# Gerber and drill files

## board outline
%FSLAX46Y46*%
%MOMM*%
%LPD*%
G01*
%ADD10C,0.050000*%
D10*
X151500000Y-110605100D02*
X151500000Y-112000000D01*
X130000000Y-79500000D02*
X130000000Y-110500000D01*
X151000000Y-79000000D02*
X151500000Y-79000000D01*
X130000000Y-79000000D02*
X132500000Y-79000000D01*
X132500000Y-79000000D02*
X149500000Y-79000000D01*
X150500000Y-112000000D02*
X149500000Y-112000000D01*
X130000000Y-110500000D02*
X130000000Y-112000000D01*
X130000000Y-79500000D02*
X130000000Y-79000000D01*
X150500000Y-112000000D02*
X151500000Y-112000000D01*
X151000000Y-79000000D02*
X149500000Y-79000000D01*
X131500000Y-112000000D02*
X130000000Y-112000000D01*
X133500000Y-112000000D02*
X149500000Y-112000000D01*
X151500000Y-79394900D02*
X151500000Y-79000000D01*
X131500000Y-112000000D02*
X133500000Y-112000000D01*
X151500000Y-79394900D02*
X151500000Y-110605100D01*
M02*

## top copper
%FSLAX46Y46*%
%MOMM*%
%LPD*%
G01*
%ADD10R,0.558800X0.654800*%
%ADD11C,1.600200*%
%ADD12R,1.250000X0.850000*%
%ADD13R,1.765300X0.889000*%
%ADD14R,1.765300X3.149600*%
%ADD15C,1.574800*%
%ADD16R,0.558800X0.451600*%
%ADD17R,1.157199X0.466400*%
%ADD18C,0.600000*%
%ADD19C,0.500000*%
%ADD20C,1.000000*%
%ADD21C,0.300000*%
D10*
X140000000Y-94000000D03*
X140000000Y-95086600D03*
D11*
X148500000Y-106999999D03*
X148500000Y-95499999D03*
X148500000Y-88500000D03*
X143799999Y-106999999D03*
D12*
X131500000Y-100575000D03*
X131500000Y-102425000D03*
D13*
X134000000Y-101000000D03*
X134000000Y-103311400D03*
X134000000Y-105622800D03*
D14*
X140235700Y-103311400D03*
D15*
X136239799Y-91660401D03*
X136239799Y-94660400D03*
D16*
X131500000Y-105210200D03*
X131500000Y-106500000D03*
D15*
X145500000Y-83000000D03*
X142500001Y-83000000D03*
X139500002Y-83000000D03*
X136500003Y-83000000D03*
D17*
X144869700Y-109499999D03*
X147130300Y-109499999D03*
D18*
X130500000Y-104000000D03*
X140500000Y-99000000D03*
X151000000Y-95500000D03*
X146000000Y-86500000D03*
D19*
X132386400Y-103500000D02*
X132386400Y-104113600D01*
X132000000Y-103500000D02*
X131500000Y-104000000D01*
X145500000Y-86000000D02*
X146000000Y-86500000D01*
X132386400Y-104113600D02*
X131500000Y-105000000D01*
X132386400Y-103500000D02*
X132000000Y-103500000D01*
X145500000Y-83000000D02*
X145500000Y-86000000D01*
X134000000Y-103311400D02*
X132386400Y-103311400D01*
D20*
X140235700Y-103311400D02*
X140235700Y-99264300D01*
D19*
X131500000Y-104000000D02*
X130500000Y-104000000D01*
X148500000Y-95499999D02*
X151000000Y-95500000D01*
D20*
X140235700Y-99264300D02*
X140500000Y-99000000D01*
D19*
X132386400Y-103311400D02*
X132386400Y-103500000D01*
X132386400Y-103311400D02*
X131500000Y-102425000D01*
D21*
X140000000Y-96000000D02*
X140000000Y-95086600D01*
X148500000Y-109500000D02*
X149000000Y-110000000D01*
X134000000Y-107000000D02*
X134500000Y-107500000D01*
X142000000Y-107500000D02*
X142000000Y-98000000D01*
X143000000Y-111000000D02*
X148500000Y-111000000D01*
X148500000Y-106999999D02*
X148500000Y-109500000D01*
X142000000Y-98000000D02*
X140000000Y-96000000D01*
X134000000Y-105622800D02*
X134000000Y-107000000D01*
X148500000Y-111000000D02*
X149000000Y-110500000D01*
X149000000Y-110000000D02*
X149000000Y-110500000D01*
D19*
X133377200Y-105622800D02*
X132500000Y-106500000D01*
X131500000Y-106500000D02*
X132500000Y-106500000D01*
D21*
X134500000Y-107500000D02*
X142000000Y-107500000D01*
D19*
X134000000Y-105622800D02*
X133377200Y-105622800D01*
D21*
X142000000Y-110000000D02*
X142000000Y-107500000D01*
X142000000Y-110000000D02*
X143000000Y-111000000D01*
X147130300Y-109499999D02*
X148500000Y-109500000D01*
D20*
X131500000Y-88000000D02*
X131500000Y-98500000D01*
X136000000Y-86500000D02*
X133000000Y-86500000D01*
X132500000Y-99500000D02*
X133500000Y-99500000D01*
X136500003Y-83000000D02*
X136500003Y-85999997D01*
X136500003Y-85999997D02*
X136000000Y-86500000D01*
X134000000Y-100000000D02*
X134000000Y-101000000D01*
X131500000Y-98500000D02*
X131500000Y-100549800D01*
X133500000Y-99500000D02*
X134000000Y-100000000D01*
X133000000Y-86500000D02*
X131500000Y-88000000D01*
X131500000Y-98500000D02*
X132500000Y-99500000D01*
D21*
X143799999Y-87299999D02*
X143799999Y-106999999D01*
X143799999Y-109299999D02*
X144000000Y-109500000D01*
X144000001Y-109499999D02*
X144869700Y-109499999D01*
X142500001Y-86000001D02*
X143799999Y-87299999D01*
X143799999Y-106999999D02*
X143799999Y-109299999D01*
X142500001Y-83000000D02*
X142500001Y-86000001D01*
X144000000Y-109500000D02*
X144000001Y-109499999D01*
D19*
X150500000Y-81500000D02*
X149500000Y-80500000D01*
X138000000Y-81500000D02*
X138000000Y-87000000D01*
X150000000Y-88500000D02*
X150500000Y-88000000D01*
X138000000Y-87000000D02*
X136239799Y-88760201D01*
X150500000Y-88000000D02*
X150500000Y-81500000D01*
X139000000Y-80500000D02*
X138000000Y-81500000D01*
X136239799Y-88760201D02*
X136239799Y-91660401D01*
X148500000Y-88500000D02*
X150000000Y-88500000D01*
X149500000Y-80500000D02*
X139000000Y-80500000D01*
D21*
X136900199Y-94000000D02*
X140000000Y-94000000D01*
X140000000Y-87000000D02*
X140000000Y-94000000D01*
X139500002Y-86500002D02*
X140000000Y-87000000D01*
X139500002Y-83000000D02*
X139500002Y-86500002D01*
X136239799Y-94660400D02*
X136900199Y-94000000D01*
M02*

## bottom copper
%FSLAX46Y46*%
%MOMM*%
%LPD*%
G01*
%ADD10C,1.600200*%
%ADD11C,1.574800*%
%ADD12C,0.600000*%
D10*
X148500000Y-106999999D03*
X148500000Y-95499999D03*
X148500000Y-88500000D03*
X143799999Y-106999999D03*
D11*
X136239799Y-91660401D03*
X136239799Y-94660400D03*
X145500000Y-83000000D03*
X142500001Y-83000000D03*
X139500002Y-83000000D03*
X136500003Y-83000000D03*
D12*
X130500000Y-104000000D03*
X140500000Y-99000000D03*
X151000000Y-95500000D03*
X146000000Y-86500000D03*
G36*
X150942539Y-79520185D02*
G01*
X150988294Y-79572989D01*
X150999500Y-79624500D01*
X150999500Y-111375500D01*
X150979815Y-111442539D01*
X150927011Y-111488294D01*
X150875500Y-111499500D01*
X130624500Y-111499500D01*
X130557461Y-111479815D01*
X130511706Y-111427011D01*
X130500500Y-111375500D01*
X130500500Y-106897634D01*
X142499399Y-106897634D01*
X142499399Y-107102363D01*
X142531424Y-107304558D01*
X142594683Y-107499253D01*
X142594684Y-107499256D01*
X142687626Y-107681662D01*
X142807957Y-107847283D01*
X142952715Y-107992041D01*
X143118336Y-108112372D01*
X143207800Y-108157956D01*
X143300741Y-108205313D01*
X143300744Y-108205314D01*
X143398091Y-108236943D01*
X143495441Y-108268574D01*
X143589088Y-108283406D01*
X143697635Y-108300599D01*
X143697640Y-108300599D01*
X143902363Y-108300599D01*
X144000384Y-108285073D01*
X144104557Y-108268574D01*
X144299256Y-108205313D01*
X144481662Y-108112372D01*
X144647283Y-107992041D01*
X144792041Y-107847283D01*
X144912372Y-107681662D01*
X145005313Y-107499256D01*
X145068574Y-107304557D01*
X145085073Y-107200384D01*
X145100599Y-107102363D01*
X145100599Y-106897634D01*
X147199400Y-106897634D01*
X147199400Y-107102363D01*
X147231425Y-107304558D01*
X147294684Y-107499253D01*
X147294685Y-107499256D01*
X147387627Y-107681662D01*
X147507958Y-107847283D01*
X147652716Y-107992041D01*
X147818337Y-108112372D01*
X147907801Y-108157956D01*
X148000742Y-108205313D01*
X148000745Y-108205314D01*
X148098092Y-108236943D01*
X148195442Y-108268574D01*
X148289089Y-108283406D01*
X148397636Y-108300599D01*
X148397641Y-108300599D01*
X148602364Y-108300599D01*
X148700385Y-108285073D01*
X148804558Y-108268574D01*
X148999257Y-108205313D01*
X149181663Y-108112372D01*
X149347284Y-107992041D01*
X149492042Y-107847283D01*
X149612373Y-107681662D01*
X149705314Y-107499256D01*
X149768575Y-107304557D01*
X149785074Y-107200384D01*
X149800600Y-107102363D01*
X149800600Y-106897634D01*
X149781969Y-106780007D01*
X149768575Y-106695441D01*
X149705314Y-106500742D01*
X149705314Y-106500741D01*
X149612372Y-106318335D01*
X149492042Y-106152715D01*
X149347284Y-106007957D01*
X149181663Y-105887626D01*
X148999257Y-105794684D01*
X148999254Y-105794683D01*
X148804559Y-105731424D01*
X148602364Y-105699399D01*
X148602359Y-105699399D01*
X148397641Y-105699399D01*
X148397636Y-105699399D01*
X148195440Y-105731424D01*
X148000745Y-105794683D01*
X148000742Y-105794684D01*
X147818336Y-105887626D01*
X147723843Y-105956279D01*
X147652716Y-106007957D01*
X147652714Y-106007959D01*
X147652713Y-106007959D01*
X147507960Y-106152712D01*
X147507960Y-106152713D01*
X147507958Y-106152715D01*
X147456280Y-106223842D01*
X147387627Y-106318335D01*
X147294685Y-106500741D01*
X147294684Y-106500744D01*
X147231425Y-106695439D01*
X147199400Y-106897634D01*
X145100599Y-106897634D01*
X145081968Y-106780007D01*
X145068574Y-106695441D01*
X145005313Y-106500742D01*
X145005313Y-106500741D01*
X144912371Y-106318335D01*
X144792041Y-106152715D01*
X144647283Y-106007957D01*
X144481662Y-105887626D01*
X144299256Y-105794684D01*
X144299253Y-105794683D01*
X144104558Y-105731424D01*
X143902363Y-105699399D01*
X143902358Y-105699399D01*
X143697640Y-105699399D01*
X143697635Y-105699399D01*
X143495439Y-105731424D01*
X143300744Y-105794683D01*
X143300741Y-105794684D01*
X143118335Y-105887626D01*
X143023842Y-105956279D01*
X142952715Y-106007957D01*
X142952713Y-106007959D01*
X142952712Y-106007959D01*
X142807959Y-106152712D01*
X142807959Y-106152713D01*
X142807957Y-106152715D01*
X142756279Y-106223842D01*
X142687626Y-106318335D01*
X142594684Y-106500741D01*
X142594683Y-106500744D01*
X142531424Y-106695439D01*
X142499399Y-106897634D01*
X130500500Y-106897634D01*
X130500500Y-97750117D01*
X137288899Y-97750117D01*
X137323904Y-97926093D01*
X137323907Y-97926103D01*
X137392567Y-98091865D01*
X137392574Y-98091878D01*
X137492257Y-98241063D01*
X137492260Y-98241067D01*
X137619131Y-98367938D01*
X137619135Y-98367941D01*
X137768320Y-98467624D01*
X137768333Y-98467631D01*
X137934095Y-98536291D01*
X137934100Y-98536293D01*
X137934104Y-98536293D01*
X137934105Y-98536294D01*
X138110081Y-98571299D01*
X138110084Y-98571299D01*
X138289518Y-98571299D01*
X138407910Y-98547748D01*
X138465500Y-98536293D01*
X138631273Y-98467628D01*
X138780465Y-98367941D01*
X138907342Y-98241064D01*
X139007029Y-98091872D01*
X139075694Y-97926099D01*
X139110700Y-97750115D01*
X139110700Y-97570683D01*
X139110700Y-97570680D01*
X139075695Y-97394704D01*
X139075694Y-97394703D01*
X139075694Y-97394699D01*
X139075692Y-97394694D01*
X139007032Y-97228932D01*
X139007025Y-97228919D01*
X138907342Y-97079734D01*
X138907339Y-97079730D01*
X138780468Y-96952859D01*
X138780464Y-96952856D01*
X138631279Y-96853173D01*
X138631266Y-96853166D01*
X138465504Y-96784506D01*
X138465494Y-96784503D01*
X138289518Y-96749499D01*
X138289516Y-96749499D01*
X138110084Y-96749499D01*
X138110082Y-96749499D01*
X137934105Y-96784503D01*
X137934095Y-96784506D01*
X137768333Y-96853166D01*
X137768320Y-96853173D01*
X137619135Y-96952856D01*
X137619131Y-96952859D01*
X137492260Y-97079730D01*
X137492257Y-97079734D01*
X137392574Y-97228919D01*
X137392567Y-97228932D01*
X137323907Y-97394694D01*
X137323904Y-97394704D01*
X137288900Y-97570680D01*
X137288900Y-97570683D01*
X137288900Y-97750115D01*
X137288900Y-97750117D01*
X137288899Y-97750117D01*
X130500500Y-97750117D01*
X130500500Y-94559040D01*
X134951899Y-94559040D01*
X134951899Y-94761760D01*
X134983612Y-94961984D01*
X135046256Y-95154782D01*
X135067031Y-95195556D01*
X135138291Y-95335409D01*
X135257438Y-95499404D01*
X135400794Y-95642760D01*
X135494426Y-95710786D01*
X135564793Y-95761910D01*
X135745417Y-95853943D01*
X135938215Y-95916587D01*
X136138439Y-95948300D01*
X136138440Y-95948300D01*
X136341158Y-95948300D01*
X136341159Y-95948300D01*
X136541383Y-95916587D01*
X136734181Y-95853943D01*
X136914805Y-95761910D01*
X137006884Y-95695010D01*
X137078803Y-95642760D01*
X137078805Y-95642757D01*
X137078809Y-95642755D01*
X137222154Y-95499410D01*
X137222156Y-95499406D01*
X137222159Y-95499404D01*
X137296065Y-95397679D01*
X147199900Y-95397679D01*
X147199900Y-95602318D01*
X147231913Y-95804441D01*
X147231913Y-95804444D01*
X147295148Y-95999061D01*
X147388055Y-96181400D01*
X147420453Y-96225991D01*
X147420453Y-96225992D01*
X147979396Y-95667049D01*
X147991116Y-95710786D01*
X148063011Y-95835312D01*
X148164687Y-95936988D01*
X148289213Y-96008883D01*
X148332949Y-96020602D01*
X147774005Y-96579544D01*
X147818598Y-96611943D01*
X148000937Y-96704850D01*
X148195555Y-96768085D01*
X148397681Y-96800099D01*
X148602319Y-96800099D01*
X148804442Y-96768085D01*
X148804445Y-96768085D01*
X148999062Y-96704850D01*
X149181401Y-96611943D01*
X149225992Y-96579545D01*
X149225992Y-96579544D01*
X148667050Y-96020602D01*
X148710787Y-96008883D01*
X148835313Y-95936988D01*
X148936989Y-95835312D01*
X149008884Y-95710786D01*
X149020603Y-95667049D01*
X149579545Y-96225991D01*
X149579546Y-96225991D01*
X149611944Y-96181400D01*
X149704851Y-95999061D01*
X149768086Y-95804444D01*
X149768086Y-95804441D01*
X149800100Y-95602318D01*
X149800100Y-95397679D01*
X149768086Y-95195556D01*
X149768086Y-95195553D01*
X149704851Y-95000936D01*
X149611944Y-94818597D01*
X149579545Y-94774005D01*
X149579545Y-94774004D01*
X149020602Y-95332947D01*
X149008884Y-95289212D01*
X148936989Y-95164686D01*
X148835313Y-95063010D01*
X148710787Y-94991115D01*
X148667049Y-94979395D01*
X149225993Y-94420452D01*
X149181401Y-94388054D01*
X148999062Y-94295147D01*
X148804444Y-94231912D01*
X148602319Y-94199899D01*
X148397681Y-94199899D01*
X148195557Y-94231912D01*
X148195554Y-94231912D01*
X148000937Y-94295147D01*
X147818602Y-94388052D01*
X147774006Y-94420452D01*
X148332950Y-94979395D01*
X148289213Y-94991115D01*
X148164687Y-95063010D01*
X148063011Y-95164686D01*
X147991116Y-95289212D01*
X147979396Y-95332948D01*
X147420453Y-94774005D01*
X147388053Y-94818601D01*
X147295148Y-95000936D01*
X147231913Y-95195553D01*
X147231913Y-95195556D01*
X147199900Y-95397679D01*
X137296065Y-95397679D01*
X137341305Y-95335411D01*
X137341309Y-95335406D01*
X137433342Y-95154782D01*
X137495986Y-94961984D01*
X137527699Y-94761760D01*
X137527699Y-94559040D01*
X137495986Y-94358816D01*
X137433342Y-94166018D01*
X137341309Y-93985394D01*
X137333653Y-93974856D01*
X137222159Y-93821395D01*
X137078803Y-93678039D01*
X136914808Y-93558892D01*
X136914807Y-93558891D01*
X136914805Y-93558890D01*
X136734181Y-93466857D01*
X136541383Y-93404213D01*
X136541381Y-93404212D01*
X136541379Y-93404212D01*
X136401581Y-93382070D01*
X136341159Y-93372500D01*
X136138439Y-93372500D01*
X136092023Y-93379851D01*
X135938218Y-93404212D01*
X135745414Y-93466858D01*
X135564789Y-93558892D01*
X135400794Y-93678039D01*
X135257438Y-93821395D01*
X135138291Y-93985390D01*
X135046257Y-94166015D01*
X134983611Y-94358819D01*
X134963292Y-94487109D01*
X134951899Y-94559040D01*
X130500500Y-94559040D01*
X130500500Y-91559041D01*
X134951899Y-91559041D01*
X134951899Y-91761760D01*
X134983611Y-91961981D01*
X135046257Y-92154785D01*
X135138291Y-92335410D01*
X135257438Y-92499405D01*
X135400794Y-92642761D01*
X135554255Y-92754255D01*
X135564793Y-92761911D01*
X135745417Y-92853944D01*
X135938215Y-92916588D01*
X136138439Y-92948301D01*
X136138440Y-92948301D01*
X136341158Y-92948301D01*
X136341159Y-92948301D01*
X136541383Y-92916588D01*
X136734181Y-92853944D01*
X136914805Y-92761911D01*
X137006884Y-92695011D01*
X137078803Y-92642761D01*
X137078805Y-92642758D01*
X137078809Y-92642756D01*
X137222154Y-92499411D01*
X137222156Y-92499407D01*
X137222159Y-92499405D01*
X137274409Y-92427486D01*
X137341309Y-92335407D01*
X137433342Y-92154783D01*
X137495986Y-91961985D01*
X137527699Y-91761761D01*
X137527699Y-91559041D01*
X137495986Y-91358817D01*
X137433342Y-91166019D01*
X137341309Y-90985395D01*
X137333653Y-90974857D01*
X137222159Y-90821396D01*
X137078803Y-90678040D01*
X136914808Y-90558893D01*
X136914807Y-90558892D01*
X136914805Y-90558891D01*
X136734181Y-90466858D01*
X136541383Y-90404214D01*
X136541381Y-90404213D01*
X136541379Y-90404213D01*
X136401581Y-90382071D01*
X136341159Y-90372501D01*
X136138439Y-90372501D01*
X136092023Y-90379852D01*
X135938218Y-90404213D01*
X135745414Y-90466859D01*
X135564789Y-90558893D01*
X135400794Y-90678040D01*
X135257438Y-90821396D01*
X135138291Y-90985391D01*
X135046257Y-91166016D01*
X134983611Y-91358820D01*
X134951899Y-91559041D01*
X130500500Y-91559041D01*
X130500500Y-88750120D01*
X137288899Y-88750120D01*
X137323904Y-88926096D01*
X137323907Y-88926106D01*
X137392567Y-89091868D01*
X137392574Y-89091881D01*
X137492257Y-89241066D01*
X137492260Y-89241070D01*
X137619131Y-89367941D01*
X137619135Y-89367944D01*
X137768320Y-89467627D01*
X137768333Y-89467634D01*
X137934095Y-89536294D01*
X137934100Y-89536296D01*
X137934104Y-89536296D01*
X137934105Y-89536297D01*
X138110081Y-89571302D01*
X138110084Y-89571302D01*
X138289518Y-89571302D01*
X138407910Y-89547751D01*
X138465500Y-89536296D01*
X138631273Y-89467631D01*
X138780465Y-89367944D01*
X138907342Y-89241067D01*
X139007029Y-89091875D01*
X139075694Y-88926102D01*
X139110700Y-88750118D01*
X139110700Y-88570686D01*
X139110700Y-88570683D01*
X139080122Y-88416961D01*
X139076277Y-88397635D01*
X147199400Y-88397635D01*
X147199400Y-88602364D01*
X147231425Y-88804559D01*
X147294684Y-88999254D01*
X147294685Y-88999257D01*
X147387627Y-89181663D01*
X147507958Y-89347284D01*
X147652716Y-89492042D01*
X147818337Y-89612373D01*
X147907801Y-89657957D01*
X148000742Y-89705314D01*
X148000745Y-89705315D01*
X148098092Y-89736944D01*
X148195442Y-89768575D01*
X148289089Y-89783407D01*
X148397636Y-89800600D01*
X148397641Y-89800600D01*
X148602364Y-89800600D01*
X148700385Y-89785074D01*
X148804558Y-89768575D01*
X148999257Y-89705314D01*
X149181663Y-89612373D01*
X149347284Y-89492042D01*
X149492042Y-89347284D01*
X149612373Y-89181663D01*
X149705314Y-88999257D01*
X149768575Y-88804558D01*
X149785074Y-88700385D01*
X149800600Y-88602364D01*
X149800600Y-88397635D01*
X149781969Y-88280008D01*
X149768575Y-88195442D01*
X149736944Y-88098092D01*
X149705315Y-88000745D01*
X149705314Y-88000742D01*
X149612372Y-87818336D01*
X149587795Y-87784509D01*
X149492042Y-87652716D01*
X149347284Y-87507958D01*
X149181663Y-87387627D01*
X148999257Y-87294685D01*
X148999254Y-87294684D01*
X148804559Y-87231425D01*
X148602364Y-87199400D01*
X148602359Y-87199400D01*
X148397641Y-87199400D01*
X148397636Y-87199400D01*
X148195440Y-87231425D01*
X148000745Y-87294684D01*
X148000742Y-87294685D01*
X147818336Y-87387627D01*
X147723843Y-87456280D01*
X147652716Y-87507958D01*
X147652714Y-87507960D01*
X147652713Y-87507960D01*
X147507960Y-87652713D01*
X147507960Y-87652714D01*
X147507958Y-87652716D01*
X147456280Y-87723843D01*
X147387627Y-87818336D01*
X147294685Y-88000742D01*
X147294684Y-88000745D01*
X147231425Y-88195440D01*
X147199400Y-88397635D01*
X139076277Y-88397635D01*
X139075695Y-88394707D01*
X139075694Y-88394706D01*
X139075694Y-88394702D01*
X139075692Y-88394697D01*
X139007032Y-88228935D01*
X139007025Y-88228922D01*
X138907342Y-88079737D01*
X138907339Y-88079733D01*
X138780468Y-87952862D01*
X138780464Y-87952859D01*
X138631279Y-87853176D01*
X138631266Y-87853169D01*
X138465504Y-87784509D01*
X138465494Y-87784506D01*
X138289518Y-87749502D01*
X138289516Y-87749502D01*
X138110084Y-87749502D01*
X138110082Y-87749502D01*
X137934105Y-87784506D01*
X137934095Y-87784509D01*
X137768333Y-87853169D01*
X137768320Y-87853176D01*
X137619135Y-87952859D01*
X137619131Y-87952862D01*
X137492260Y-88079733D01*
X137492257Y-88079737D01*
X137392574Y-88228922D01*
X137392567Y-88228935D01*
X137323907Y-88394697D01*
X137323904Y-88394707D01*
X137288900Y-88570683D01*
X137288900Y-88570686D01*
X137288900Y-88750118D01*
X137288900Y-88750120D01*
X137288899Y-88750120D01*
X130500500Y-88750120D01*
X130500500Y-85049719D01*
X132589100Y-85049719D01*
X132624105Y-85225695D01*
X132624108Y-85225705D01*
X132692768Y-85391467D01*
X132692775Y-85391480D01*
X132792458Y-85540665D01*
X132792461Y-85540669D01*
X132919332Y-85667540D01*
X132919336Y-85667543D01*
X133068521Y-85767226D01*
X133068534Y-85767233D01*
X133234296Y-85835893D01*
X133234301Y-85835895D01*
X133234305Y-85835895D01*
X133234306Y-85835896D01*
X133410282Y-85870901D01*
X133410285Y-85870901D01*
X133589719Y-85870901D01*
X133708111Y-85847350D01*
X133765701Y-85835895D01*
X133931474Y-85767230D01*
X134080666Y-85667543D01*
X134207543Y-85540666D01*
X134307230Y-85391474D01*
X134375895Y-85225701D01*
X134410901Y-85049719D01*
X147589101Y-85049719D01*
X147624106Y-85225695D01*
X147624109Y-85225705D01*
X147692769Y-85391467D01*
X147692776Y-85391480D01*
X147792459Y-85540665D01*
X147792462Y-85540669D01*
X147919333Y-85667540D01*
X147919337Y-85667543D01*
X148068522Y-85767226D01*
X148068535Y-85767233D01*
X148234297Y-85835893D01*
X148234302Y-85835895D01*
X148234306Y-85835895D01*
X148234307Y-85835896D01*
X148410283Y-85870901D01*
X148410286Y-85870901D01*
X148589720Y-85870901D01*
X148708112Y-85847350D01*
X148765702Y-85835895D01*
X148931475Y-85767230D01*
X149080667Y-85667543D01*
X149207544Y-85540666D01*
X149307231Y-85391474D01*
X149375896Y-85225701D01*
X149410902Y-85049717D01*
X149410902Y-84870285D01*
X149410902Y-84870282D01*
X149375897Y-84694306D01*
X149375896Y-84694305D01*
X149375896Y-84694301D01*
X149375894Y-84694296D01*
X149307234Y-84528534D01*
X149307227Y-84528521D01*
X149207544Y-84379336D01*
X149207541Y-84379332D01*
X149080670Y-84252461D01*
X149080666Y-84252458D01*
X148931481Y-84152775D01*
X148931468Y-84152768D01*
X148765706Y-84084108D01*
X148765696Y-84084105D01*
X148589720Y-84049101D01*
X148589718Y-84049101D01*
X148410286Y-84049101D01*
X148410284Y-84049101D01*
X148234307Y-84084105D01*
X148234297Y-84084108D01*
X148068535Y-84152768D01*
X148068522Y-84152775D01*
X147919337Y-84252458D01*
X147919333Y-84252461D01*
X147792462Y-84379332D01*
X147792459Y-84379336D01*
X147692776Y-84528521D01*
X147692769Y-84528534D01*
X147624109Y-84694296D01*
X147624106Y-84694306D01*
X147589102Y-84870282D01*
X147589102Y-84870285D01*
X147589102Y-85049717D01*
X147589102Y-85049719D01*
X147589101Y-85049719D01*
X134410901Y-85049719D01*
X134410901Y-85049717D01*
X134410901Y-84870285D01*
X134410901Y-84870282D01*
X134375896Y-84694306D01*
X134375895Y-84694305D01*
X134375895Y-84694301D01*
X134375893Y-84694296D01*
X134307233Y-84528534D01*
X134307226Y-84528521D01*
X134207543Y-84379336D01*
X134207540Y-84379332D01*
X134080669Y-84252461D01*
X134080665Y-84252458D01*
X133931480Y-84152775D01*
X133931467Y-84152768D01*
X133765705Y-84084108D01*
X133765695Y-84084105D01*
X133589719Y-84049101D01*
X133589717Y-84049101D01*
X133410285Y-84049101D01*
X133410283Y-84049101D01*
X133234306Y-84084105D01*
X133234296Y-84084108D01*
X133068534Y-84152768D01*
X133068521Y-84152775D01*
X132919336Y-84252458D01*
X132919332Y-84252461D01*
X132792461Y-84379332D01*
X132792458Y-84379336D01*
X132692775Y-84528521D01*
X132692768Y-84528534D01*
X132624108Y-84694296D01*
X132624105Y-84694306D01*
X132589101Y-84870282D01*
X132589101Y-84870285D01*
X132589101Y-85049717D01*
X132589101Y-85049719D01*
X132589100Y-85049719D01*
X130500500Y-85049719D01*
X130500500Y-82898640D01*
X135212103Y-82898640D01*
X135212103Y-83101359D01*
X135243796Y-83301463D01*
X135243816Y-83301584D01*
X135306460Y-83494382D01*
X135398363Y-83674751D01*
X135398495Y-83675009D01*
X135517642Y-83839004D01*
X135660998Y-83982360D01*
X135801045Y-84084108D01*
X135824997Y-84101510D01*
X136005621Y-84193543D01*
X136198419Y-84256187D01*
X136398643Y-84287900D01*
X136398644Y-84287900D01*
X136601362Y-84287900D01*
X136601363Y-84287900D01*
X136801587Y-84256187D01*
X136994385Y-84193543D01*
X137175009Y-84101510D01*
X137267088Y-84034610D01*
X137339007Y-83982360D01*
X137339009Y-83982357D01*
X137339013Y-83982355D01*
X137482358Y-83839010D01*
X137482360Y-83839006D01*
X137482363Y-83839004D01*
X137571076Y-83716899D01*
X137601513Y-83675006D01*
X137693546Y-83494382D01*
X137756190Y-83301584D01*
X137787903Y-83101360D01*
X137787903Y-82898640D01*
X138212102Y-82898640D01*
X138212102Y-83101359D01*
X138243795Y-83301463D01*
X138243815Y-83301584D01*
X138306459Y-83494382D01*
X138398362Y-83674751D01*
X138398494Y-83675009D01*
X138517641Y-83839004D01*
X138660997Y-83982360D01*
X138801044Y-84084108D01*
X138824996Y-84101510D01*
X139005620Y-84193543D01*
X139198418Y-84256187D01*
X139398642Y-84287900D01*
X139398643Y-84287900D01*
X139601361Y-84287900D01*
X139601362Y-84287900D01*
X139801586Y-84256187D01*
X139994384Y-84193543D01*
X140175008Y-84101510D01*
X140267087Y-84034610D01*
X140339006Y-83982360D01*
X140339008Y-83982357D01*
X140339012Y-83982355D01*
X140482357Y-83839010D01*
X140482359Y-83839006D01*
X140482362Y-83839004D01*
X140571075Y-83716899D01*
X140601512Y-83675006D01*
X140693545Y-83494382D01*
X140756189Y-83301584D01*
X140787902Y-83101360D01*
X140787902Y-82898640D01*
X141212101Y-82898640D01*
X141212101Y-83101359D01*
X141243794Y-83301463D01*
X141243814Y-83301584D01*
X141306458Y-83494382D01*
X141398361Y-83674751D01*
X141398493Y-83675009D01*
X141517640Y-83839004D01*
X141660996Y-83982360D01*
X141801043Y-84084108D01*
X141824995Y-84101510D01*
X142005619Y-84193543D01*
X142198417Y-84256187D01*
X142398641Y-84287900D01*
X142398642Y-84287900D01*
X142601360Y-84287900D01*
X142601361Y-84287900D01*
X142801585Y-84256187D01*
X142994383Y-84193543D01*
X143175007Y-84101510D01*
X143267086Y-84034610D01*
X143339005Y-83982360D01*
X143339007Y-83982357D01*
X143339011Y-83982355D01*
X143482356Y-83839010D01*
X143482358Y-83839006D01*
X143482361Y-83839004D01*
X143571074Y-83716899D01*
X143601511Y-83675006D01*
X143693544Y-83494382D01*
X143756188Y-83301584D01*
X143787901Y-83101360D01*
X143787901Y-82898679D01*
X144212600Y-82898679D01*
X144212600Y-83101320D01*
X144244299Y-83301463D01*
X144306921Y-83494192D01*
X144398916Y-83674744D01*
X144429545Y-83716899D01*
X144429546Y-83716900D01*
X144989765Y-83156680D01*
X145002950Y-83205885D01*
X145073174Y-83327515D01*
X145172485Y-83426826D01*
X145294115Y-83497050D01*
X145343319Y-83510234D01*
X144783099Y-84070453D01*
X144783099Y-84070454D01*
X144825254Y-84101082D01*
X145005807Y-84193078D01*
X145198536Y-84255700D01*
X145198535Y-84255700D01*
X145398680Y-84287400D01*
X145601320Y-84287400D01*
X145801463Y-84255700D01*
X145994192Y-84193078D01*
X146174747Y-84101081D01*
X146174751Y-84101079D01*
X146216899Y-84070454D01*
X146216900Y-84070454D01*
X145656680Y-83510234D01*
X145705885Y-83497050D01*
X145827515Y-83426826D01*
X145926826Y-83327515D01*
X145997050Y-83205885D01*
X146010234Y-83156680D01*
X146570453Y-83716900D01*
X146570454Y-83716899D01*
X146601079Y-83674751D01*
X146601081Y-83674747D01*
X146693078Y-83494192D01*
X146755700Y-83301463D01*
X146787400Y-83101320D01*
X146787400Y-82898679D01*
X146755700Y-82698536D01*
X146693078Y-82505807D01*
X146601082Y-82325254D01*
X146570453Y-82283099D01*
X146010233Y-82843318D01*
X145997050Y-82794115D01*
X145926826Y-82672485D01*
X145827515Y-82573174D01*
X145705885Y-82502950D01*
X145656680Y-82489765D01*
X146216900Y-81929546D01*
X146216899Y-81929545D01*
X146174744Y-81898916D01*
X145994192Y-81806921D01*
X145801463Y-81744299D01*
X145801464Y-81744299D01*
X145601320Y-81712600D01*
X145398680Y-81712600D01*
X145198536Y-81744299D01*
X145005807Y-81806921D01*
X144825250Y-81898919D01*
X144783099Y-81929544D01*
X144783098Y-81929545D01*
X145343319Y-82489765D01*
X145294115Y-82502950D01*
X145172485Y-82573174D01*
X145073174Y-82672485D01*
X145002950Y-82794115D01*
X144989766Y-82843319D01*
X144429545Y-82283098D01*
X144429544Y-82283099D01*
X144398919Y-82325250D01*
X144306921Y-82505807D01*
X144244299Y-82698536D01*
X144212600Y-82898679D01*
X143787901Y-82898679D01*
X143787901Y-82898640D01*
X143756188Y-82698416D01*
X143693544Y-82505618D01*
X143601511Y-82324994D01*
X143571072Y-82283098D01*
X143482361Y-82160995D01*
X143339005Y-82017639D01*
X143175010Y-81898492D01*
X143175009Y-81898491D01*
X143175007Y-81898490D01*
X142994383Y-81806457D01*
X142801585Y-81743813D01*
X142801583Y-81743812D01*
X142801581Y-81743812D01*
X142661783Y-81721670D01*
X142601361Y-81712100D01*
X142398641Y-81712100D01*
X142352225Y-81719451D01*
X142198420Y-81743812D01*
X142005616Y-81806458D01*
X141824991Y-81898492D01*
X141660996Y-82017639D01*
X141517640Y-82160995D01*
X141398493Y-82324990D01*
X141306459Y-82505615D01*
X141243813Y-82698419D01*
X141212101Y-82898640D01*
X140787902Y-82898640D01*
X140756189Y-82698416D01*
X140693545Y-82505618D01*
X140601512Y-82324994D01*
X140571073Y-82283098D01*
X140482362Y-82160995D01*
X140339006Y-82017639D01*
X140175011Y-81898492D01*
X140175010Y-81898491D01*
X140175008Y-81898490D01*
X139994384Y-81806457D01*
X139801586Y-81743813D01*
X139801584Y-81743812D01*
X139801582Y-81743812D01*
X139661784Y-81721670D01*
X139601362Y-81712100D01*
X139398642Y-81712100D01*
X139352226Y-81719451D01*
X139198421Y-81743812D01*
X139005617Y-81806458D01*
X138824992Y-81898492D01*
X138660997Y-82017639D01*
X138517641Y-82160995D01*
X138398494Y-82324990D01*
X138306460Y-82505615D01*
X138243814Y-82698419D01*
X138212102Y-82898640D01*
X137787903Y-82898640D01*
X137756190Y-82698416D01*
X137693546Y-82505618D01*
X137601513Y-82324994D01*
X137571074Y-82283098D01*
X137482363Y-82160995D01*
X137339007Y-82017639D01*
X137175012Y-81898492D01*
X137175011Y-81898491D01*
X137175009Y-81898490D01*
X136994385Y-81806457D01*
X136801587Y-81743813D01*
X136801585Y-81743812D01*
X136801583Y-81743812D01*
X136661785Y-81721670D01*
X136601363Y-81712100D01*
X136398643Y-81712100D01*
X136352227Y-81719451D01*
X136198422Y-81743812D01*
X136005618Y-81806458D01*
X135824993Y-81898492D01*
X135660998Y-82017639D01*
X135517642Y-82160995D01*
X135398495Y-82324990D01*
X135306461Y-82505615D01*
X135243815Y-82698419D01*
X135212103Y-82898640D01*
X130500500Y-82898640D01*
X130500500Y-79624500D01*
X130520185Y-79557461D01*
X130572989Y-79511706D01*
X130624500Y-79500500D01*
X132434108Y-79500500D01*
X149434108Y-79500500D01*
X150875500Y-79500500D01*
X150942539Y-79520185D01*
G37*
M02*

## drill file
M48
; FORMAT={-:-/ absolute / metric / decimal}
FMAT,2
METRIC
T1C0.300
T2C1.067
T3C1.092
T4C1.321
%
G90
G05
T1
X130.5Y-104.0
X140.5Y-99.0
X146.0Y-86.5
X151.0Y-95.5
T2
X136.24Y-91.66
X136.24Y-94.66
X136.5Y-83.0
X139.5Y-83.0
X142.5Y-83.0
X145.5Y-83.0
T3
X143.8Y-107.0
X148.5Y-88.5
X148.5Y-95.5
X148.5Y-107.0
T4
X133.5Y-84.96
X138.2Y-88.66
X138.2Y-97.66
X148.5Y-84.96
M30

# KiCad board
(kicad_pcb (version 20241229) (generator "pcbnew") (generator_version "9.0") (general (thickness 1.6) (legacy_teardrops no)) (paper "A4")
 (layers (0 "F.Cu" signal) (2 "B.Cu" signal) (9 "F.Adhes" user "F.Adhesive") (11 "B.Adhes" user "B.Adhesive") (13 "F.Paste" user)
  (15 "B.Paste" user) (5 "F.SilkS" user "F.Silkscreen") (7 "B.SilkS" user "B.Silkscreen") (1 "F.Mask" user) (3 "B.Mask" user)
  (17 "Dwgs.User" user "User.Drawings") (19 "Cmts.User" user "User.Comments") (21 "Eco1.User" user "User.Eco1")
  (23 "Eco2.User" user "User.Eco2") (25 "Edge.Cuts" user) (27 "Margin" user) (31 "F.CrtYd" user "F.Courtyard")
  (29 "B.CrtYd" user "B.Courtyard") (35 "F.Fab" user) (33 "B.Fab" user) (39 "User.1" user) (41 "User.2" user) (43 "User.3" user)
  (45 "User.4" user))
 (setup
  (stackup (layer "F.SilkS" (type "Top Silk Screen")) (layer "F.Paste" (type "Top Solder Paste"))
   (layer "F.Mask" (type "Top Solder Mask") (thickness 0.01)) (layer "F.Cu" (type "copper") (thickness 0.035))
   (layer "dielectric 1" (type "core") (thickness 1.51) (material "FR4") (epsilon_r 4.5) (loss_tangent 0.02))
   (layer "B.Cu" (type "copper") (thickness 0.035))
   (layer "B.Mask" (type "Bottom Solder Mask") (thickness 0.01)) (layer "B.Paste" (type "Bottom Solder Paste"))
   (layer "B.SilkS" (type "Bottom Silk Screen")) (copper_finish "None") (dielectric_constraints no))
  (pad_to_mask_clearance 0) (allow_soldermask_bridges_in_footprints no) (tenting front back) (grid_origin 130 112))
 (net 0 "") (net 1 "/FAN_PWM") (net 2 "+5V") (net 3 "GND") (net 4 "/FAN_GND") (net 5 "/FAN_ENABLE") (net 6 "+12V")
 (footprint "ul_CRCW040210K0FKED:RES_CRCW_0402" (layer "F.Cu") (at 140 94.5433 -90)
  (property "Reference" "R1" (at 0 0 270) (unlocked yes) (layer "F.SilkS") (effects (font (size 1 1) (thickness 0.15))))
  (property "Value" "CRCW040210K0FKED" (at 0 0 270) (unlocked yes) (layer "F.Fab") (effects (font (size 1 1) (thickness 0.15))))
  (pad "1" smd rect (at -0.5433 0 270) (size 0.6548 0.5588) (layers "F.Cu" "F.Mask" "F.Paste") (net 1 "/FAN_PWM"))
  (pad "2" smd rect (at 0.5433 0 270) (size 0.6548 0.5588) (layers "F.Cu" "F.Mask" "F.Paste") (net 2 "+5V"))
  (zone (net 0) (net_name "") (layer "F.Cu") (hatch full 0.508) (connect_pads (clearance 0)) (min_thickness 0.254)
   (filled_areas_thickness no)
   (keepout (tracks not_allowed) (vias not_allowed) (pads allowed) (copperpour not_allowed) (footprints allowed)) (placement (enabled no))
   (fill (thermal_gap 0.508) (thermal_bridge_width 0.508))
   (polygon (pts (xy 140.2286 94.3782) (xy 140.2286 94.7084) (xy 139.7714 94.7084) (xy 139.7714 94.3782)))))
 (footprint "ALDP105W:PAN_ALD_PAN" (layer "F.Cu") (at 148.5 106.999999 180)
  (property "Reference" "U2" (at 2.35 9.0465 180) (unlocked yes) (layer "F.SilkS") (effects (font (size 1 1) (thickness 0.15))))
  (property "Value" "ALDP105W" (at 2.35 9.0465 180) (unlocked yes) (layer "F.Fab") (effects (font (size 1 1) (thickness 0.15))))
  (pad "1" thru_hole circle (at 0 0 180) (size 1.6002 1.6002) (drill 1.0922) (layers "*.Cu" "*.Mask") (remove_unused_layers no)
   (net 2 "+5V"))
  (pad "2" thru_hole circle (at 0 11.5 180) (size 1.6002 1.6002) (drill 1.0922) (layers "*.Cu" "*.Mask") (remove_unused_layers no)
   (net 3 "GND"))
  (pad "3" thru_hole circle (at 0 18.499999 180) (size 1.6002 1.6002) (drill 1.0922) (layers "*.Cu" "*.Mask") (remove_unused_layers no)
   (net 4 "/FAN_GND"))
  (pad "4" thru_hole circle (at 4.700001 0 180) (size 1.6002 1.6002) (drill 1.0922) (layers "*.Cu" "*.Mask") (remove_unused_layers no)
   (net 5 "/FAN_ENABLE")))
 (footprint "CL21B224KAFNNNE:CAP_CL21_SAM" (layer "F.Cu") (at 131.5 101.5 -90)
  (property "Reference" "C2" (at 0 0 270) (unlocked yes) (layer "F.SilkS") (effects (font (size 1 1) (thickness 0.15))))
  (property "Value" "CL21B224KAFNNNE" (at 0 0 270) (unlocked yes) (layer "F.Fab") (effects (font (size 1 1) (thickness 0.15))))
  (pad "1" smd rect (at -0.925 0 270) (size 0.85 1.25) (layers "F.Cu" "F.Mask" "F.Paste") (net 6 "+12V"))
  (pad "2" smd rect (at 0.925 0 270) (size 0.85 1.25) (layers "F.Cu" "F.Mask" "F.Paste") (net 3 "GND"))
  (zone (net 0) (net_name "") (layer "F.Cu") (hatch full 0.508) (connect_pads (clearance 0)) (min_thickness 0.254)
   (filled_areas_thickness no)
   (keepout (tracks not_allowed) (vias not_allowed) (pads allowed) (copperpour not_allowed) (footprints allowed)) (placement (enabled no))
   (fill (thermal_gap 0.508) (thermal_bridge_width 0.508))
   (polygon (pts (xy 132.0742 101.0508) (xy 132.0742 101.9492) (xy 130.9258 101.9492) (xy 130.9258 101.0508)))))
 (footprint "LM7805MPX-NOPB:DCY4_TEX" (layer "F.Cu") (at 137.11785 103.3114 -90)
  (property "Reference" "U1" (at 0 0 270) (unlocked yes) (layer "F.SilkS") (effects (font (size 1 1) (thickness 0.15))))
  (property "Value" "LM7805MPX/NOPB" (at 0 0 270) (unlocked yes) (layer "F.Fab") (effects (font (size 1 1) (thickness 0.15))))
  (pad "1" smd rect (at -2.3114 3.11785 270) (size 0.889 1.7653) (layers "F.Cu" "F.Mask" "F.Paste") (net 6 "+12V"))
  (pad "2" smd rect (at 0 3.11785 270) (size 0.889 1.7653) (layers "F.Cu" "F.Mask" "F.Paste") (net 3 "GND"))
  (pad "3" smd rect (at 2.3114 3.11785 270) (size 0.889 1.7653) (layers "F.Cu" "F.Mask" "F.Paste") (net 2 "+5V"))
  (pad "4" smd rect (at 0 -3.11785 270) (size 3.1496 1.7653) (layers "F.Cu" "F.Mask" "F.Paste") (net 3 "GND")))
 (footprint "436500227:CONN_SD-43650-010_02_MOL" (layer "F.Cu") (at 136.239799 91.660401 90)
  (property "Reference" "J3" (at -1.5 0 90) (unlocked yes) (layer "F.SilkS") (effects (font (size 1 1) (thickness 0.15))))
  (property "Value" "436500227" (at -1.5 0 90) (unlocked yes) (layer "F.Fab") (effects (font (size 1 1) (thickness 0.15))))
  (pad "" np_thru_hole circle (at -5.999998 1.960001 90) (size 1.3208 1.3208) (drill 1.3208) (layers "*.Cu" "*.Mask"))
  (pad "" np_thru_hole circle (at 2.999999 1.960001 90) (size 1.3208 1.3208) (drill 1.3208) (layers "*.Cu" "*.Mask"))
  (pad "1" thru_hole circle (at 0 0 90) (size 1.5748 1.5748) (drill 1.0668) (layers "*.Cu" "*.Mask") (remove_unused_layers no)
   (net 4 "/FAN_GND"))
  (pad "2" thru_hole circle (at -2.999999 0 90) (size 1.5748 1.5748) (drill 1.0668) (layers "*.Cu" "*.Mask") (remove_unused_layers no)
   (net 1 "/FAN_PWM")))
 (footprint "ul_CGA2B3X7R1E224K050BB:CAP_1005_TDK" (layer "F.Cu") (at 131.5 105.8551 -90)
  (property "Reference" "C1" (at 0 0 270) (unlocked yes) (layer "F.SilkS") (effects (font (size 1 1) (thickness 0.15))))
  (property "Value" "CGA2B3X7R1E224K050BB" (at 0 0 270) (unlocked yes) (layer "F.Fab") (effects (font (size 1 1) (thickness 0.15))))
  (pad "1" smd rect (at -0.6449 0 270) (size 0.4516 0.5588) (layers "F.Cu" "F.Mask" "F.Paste") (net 3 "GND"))
  (pad "2" smd rect (at 0.6449 0 270) (size 0.4516 0.5588) (layers "F.Cu" "F.Mask" "F.Paste") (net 2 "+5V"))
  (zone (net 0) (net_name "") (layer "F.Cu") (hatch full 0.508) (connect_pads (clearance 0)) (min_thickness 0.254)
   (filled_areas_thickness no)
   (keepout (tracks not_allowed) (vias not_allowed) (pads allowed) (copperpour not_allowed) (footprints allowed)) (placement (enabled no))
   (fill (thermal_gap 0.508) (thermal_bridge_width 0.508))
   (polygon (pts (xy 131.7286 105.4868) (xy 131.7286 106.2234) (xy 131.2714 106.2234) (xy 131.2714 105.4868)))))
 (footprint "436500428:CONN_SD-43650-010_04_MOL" (layer "F.Cu") (at 145.5 83)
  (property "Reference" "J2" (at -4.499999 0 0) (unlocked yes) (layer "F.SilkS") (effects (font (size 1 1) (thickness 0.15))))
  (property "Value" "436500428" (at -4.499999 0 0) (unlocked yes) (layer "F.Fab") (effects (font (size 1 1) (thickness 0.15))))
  (pad "" np_thru_hole circle (at -11.999999 1.960001) (size 1.3208 1.3208) (drill 1.3208) (layers "*.Cu" "*.Mask"))
  (pad "" np_thru_hole circle (at 3.000002 1.960001) (size 1.3208 1.3208) (drill 1.3208) (layers "*.Cu" "*.Mask"))
  (pad "1" thru_hole circle (at 0 0) (size 1.5748 1.5748) (drill 1.0668) (layers "*.Cu" "*.Mask") (remove_unused_layers no) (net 3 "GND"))
  (pad "2" thru_hole circle (at -2.999999 0) (size 1.5748 1.5748) (drill 1.0668) (layers "*.Cu" "*.Mask") (remove_unused_layers no)
   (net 5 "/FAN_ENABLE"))
  (pad "3" thru_hole circle (at -5.999998 0) (size 1.5748 1.5748) (drill 1.0668) (layers "*.Cu" "*.Mask") (remove_unused_layers no)
   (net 1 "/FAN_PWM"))
  (pad "4" thru_hole circle (at -8.999997 0) (size 1.5748 1.5748) (drill 1.0668) (layers "*.Cu" "*.Mask") (remove_unused_layers no)
   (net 6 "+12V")))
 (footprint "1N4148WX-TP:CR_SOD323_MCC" (layer "F.Cu") (at 146 109.499999)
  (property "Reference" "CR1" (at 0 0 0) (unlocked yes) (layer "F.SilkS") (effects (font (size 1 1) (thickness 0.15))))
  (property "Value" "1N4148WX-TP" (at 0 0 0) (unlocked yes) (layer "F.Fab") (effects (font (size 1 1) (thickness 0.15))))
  (pad "1" smd rect (at -1.1303 0) (size 1.157199 0.4664) (layers "F.Cu" "F.Mask" "F.Paste") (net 5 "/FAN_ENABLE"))
  (pad "2" smd rect (at 1.1303 0) (size 1.157199 0.4664) (layers "F.Cu" "F.Mask" "F.Paste") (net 2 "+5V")))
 (gr_line (start 151.5 110.6051) (end 151.5 112) (stroke (width 0.05) (type default)) (layer "Edge.Cuts"))
 (gr_line (start 130 79.5) (end 130 110.5) (stroke (width 0.05) (type default)) (layer "Edge.Cuts"))
 (gr_line (start 151 79) (end 151.5 79) (stroke (width 0.05) (type default)) (layer "Edge.Cuts"))
 (gr_line (start 130 79) (end 132.5 79) (stroke (width 0.05) (type default)) (layer "Edge.Cuts"))
 (gr_line (start 132.5 79) (end 149.5 79) (stroke (width 0.05) (type default)) (layer "Edge.Cuts"))
 (gr_line (start 150.5 112) (end 149.5 112) (stroke (width 0.05) (type default)) (layer "Edge.Cuts"))
 (gr_line (start 130 110.5) (end 130 112) (stroke (width 0.05) (type default)) (layer "Edge.Cuts"))
 (gr_line (start 130 79.5) (end 130 79) (stroke (width 0.05) (type default)) (layer "Edge.Cuts"))
 (gr_line (start 150.5 112) (end 151.5 112) (stroke (width 0.05) (type default)) (layer "Edge.Cuts"))
 (gr_line (start 151 79) (end 149.5 79) (stroke (width 0.05) (type default)) (layer "Edge.Cuts"))
 (gr_line (start 131.5 112) (end 130 112) (stroke (width 0.05) (type default)) (layer "Edge.Cuts"))
 (gr_line (start 133.5 112) (end 149.5 112) (stroke (width 0.05) (type default)) (layer "Edge.Cuts"))
 (gr_line (start 151.5 79.3949) (end 151.5 79) (stroke (width 0.05) (type default)) (layer "Edge.Cuts"))
 (gr_line (start 131.5 112) (end 133.5 112) (stroke (width 0.05) (type default)) (layer "Edge.Cuts"))
 (gr_line (start 151.5 79.3949) (end 151.5 110.6051) (stroke (width 0.05) (type solid)) (layer "Edge.Cuts"))
 (segment (start 132.3864 103.5) (end 132.3864 104.1136) (width 0.5) (layer "F.Cu") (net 3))
 (segment (start 132 103.5) (end 131.5 104) (width 0.5) (layer "F.Cu") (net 3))
 (segment (start 145.5 86) (end 146 86.5) (width 0.5) (layer "F.Cu") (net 3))
 (segment (start 132.3864 104.1136) (end 131.5 105) (width 0.5) (layer "F.Cu") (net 3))
 (segment (start 132.3864 103.5) (end 132 103.5) (width 0.5) (layer "F.Cu") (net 3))
 (segment (start 145.5 83) (end 145.5 86) (width 0.5) (layer "F.Cu") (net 3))
 (segment (start 134 103.3114) (end 132.3864 103.3114) (width 0.5) (layer "F.Cu") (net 3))
 (segment (start 140.2357 103.3114) (end 140.2357 99.2643) (width 1) (layer "F.Cu") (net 3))
 (segment (start 131.5 104) (end 130.5 104) (width 0.5) (layer "F.Cu") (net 3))
 (segment (start 148.5 95.499999) (end 151 95.5) (width 0.5) (layer "F.Cu") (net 3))
 (segment (start 140.2357 99.2643) (end 140.5 99) (width 1) (layer "F.Cu") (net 3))
 (segment (start 132.3864 103.3114) (end 132.3864 103.5) (width 0.5) (layer "F.Cu") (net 3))
 (segment (start 132.3864 103.3114) (end 131.5 102.425) (width 0.5) (layer "F.Cu") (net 3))
 (via (at 130.5 104) (size 0.6) (drill 0.3) (layers "F.Cu" "B.Cu") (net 3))
 (via (at 140.5 99) (size 0.6) (drill 0.3) (layers "F.Cu" "B.Cu") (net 3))
 (via (at 151 95.5) (size 0.6) (drill 0.3) (layers "F.Cu" "B.Cu") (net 3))
 (via (at 146 86.5) (size 0.6) (drill 0.3) (layers "F.Cu" "B.Cu") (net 3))
 (segment (start 140 96) (end 140 95.0866) (width 0.3) (layer "F.Cu") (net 2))
 (segment (start 148.5 109.5) (end 149 110) (width 0.3) (layer "F.Cu") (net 2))
 (segment (start 134 107) (end 134.5 107.5) (width 0.3) (layer "F.Cu") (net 2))
 (segment (start 142 107.5) (end 142 98) (width 0.3) (layer "F.Cu") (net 2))
 (segment (start 143 111) (end 148.5 111) (width 0.3) (layer "F.Cu") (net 2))
 (segment (start 148.5 106.999999) (end 148.5 109.5) (width 0.3) (layer "F.Cu") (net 2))
 (segment (start 142 98) (end 140 96) (width 0.3) (layer "F.Cu") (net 2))
 (segment (start 134 105.6228) (end 134 107) (width 0.3) (layer "F.Cu") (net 2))
 (segment (start 148.5 111) (end 149 110.5) (width 0.3) (layer "F.Cu") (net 2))
 (segment (start 149 110) (end 149 110.5) (width 0.3) (layer "F.Cu") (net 2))
 (segment (start 133.3772 105.6228) (end 132.5 106.5) (width 0.5) (layer "F.Cu") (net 2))
 (segment (start 131.5 106.5) (end 132.5 106.5) (width 0.5) (layer "F.Cu") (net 2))
 (segment (start 134.5 107.5) (end 142 107.5) (width 0.3) (layer "F.Cu") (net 2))
 (segment (start 134 105.6228) (end 133.3772 105.6228) (width 0.5) (layer "F.Cu") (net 2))
 (segment (start 142 110) (end 142 107.5) (width 0.3) (layer "F.Cu") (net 2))
 (segment (start 142 110) (end 143 111) (width 0.3) (layer "F.Cu") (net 2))
 (segment (start 147.1303 109.499999) (end 148.5 109.5) (width 0.3) (layer "F.Cu") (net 2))
 (segment (start 131.5 88) (end 131.5 98.5) (width 1) (layer "F.Cu") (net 6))
 (segment (start 136 86.5) (end 133 86.5) (width 1) (layer "F.Cu") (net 6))
 (segment (start 132.5 99.5) (end 133.5 99.5) (width 1) (layer "F.Cu") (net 6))
 (segment (start 136.500003 83) (end 136.500003 85.999997) (width 1) (layer "F.Cu") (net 6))
 (segment (start 136.500003 85.999997) (end 136 86.5) (width 1) (layer "F.Cu") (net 6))
 (segment (start 134 100) (end 134 101) (width 1) (layer "F.Cu") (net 6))
 (segment (start 131.5 98.5) (end 131.5 100.5498) (width 1) (layer "F.Cu") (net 6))
 (segment (start 133.5 99.5) (end 134 100) (width 1) (layer "F.Cu") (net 6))
 (segment (start 133 86.5) (end 131.5 88) (width 1) (layer "F.Cu") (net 6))
 (segment (start 131.5 98.5) (end 132.5 99.5) (width 1) (layer "F.Cu") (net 6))
 (segment (start 143.799999 87.299999) (end 143.799999 106.999999) (width 0.3) (layer "F.Cu") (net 5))
 (segment (start 143.799999 109.299999) (end 144 109.5) (width 0.3) (layer "F.Cu") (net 5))
 (segment (start 144.000001 109.499999) (end 144.8697 109.499999) (width 0.3) (layer "F.Cu") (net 5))
 (segment (start 142.500001 86.000001) (end 143.799999 87.299999) (width 0.3) (layer "F.Cu") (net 5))
 (segment (start 143.799999 106.999999) (end 143.799999 109.299999) (width 0.3) (layer "F.Cu") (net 5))
 (segment (start 142.500001 83) (end 142.500001 86.000001) (width 0.3) (layer "F.Cu") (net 5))
 (segment (start 144 109.5) (end 144.000001 109.499999) (width 0.3) (layer "F.Cu") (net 5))
 (segment (start 150.5 81.5) (end 149.5 80.5) (width 0.5) (layer "F.Cu") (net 4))
 (segment (start 138 81.5) (end 138 87) (width 0.5) (layer "F.Cu") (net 4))
 (segment (start 150 88.5) (end 150.5 88) (width 0.5) (layer "F.Cu") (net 4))
 (segment (start 138 87) (end 136.239799 88.760201) (width 0.5) (layer "F.Cu") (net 4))
 (segment (start 150.5 88) (end 150.5 81.5) (width 0.5) (layer "F.Cu") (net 4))
 (segment (start 139 80.5) (end 138 81.5) (width 0.5) (layer "F.Cu") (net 4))
 (segment (start 136.239799 88.760201) (end 136.239799 91.660401) (width 0.5) (layer "F.Cu") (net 4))
 (segment (start 148.5 88.5) (end 150 88.5) (width 0.5) (layer "F.Cu") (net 4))
 (segment (start 149.5 80.5) (end 139 80.5) (width 0.5) (layer "F.Cu") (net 4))
 (segment (start 136.900199 94) (end 140 94) (width 0.3) (layer "F.Cu") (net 1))
 (segment (start 140 87) (end 140 94) (width 0.3) (layer "F.Cu") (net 1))
 (segment (start 139.500002 86.500002) (end 140 87) (width 0.3) (layer "F.Cu") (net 1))
 (segment (start 139.500002 83) (end 139.500002 86.500002) (width 0.3) (layer "F.Cu") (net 1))
 (segment (start 136.239799 94.6604) (end 136.900199 94) (width 0.3) (layer "F.Cu") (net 1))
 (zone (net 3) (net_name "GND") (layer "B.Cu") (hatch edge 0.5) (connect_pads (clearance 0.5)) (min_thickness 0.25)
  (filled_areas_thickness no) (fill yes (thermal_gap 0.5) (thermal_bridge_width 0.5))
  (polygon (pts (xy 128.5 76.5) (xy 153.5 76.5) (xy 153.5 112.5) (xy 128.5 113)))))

